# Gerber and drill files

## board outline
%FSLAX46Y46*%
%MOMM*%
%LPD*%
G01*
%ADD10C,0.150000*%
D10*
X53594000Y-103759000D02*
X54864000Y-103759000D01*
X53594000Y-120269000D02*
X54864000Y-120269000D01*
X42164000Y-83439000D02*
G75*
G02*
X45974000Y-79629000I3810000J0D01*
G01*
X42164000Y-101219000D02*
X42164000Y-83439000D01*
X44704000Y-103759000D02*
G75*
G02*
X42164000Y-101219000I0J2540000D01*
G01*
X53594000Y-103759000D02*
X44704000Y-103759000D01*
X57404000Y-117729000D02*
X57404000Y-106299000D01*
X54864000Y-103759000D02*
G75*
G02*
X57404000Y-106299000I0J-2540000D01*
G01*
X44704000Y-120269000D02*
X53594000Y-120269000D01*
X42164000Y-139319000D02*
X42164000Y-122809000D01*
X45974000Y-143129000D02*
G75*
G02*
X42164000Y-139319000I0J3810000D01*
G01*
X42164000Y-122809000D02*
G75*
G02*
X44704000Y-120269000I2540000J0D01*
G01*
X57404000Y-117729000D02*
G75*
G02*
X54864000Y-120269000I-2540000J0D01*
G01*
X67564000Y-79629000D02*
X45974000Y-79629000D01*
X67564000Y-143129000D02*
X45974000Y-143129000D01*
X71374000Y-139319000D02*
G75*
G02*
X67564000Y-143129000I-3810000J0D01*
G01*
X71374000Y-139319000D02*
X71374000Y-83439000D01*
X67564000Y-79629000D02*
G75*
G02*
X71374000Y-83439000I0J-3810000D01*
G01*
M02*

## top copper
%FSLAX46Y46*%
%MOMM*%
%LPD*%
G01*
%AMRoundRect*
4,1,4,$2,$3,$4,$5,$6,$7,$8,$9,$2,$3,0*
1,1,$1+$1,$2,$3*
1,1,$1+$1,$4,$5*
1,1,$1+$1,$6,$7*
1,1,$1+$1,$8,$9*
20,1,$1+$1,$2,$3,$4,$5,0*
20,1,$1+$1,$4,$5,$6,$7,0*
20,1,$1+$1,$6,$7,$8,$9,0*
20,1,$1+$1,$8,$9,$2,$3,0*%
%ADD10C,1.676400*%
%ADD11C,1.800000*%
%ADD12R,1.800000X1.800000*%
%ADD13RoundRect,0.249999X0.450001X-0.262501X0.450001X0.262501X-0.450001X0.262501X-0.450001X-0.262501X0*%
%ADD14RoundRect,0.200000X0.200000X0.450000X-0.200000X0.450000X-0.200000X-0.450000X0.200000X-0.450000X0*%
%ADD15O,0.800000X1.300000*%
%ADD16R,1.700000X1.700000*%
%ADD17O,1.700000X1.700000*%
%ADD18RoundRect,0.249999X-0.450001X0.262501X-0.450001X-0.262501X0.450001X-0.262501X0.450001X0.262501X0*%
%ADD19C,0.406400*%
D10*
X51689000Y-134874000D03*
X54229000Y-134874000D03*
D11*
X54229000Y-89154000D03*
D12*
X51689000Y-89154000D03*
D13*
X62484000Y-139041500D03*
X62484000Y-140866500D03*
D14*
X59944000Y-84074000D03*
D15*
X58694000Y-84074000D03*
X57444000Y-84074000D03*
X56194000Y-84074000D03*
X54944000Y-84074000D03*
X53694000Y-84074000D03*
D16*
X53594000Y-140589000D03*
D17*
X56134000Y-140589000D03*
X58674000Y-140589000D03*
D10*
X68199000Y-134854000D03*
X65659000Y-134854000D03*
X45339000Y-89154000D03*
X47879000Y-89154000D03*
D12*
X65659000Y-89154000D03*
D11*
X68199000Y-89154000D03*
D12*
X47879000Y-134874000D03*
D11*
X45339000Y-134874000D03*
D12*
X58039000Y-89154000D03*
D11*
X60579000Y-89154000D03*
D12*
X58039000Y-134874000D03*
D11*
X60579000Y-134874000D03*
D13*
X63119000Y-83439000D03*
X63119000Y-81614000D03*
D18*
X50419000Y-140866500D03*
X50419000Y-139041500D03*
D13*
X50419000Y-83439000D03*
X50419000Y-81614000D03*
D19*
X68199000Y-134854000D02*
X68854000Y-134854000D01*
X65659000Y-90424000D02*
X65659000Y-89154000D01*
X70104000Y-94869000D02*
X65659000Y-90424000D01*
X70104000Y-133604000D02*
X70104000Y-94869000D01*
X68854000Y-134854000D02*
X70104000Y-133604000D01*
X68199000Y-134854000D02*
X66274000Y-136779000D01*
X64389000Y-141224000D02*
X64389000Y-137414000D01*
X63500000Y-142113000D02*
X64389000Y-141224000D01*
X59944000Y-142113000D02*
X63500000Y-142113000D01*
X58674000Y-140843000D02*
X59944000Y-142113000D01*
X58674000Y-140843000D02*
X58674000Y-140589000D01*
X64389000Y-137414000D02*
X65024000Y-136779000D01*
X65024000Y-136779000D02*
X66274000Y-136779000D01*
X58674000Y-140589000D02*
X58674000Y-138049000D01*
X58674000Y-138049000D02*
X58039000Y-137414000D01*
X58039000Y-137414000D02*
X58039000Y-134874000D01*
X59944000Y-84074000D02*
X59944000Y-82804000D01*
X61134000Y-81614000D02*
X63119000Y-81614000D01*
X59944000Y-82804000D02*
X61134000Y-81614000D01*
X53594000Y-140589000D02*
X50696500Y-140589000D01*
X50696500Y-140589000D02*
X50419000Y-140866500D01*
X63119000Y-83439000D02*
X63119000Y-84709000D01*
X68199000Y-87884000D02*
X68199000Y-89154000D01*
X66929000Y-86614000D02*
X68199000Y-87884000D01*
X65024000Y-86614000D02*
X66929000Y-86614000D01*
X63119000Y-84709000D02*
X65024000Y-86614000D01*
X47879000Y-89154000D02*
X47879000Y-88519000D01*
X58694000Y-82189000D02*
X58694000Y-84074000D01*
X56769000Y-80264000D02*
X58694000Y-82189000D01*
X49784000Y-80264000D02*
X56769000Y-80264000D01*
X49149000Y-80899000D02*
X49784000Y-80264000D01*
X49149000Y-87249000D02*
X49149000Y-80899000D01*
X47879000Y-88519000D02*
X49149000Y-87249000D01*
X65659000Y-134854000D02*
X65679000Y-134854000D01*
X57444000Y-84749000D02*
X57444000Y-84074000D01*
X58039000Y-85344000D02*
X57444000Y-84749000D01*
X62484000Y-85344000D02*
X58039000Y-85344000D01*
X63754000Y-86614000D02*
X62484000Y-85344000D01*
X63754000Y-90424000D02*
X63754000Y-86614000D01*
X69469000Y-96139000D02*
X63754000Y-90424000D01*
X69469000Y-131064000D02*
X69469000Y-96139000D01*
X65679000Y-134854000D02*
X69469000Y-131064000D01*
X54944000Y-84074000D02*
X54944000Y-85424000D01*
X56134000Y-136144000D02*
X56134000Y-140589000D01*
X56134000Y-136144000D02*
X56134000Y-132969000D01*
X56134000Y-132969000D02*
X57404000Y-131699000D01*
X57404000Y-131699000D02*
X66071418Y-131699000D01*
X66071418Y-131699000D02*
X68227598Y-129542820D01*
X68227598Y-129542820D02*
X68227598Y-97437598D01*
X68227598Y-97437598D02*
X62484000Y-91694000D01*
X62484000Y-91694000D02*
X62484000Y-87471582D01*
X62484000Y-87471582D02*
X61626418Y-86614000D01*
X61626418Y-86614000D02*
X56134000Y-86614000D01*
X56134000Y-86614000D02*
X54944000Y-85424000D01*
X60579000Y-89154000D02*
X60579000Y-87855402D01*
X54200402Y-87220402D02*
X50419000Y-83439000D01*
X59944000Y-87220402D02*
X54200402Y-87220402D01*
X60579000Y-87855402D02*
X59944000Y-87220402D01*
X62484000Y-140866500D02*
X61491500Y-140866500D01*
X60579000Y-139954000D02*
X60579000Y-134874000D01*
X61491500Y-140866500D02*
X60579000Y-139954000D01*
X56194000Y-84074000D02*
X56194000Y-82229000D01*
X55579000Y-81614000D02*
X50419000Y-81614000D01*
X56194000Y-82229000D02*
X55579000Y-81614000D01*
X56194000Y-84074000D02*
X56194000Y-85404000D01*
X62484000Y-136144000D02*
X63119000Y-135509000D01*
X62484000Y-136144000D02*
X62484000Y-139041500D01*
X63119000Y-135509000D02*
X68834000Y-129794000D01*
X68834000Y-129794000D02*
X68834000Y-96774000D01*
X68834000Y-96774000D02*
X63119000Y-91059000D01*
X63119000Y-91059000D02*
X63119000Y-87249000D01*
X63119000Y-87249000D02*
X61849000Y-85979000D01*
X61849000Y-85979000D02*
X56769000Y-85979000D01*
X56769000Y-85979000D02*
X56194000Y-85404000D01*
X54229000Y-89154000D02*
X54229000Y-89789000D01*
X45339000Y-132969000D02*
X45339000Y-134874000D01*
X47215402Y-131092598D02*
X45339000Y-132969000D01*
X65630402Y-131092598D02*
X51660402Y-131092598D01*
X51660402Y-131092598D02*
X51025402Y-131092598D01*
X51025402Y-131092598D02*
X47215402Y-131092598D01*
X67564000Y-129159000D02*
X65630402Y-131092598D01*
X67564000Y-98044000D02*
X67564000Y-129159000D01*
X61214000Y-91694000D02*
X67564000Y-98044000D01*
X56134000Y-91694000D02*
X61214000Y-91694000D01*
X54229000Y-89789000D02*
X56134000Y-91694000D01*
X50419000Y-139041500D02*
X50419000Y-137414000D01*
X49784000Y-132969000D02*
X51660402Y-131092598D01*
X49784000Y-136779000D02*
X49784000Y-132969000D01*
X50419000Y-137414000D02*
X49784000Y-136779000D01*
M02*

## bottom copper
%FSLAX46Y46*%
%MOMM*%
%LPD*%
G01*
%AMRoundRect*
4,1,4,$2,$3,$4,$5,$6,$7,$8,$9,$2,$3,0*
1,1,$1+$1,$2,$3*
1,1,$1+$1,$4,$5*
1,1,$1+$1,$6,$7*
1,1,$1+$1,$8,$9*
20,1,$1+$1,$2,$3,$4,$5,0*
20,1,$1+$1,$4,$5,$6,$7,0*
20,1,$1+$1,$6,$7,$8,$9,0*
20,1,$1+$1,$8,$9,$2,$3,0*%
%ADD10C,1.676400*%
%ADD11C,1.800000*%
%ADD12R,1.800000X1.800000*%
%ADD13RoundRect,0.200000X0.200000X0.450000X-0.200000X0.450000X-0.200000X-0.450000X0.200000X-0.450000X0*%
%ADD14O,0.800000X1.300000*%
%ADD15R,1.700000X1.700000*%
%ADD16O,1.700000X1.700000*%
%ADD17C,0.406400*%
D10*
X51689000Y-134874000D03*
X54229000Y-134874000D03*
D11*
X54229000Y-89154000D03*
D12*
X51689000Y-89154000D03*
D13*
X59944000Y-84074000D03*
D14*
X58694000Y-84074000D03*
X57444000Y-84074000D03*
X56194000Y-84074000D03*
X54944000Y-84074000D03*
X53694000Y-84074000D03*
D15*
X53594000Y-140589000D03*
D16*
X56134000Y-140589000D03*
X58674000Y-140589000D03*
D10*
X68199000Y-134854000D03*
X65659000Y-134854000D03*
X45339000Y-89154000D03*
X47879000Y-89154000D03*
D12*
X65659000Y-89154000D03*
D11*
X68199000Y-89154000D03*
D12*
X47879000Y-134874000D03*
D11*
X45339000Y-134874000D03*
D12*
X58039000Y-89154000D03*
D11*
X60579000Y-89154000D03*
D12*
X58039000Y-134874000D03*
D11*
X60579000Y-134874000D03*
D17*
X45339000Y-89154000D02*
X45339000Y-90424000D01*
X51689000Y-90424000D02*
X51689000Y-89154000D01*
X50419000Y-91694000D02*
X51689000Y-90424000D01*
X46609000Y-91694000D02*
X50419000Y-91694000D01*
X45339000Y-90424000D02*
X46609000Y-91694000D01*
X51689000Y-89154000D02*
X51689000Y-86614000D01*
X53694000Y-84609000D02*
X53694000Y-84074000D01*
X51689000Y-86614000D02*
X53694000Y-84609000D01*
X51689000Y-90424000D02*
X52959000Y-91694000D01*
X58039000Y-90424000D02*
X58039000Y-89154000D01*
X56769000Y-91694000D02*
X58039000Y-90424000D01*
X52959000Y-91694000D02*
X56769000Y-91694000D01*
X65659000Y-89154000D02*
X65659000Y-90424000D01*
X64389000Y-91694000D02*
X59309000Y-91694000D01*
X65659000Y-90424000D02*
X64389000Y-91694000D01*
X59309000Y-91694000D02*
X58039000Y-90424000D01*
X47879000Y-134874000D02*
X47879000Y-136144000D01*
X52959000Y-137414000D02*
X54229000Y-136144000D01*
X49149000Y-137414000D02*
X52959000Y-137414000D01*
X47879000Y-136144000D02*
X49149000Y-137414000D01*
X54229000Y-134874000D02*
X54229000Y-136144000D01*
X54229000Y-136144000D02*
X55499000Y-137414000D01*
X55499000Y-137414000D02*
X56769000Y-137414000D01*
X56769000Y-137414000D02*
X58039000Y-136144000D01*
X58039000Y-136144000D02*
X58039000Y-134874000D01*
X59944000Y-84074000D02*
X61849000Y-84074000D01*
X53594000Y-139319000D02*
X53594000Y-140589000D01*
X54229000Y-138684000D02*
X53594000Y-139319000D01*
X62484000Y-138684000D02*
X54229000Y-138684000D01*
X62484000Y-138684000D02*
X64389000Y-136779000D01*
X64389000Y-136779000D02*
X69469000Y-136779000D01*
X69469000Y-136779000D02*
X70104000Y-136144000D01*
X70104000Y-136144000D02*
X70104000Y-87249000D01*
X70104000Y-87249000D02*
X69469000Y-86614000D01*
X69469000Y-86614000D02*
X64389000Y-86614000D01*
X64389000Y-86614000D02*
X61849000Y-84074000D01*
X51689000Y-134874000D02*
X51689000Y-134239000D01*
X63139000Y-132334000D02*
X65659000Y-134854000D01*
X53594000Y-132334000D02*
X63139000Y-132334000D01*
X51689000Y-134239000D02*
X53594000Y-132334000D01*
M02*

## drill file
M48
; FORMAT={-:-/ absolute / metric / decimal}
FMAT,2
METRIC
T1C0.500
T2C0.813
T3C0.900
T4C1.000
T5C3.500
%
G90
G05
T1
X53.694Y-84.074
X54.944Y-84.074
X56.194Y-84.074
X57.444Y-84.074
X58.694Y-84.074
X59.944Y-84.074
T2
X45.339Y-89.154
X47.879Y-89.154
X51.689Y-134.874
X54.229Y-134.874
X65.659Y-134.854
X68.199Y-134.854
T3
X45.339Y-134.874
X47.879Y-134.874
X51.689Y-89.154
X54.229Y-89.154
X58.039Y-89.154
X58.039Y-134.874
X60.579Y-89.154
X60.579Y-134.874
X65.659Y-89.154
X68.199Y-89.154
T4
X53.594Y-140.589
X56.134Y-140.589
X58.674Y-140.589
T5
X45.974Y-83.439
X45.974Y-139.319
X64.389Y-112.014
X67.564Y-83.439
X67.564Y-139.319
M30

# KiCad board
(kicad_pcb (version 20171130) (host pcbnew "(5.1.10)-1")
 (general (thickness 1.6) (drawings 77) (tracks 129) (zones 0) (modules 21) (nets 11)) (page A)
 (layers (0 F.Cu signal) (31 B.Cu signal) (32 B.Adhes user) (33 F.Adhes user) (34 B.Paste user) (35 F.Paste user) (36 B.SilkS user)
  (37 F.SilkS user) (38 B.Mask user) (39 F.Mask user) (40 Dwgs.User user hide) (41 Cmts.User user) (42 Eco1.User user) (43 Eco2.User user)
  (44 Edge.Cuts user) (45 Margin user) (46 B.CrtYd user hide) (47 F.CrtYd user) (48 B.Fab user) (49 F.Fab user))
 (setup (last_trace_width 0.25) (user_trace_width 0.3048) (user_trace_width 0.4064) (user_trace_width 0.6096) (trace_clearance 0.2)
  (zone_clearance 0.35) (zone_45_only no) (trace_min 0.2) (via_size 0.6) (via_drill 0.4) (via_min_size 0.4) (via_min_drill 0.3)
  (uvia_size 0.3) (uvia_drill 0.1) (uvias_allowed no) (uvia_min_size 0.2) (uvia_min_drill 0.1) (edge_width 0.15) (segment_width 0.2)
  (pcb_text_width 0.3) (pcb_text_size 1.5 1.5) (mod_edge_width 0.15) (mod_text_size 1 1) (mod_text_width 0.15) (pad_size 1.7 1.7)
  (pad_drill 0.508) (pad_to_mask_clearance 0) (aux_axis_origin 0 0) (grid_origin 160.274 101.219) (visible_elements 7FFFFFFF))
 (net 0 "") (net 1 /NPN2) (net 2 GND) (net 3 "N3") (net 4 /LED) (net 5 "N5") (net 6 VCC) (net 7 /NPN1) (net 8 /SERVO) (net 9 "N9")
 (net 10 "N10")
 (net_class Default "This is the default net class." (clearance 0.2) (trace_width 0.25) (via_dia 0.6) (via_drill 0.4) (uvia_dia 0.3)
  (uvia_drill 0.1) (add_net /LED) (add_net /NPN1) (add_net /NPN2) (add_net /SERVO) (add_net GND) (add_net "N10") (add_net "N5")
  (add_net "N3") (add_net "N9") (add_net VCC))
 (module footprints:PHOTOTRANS (layer F.Cu) (at 52.959 134.874 180)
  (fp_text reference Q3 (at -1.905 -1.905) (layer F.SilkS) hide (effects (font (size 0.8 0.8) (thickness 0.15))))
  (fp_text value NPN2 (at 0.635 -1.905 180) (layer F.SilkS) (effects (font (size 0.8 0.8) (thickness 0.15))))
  (pad 1 thru_hole circle (at 1.27 0 225) (size 1.6764 1.6764) (drill 0.8128) (layers *.Cu *.Mask F.SilkS) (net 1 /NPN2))
  (pad 2 thru_hole circle (at -1.27 0 180) (size 1.6764 1.6764) (drill 0.8128) (layers *.Cu *.Mask F.SilkS) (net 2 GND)))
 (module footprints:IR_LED (layer F.Cu) (at 51.689 89.154)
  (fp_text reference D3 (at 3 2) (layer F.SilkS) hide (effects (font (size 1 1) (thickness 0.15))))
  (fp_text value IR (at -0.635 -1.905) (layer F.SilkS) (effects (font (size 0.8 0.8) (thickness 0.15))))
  (pad 2 thru_hole circle (at 2.54 0) (size 1.8 1.8) (drill 0.9) (layers *.Cu *.Mask) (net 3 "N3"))
  (pad 1 thru_hole rect (at 0 0) (size 1.8 1.8) (drill 0.9) (layers *.Cu *.Mask) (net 2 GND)))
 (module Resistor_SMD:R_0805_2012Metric (layer F.Cu) (at 62.484 139.954 90)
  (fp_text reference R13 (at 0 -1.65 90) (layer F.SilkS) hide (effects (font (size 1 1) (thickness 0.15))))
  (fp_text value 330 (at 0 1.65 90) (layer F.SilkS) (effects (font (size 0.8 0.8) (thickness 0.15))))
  (pad 2 smd roundrect (at 0.9125 0 90) (size 1.025 1.4) (layers F.Cu F.Paste F.Mask) (roundrect_rratio 0.2439014634146341) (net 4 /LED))
  (pad 1 smd roundrect (at -0.9125 0 90) (size 1.025 1.4) (layers F.Cu F.Paste F.Mask) (roundrect_rratio 0.2439014634146341) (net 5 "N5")))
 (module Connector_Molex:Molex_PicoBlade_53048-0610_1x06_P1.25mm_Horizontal (layer F.Cu) (at 59.944 84.074 180)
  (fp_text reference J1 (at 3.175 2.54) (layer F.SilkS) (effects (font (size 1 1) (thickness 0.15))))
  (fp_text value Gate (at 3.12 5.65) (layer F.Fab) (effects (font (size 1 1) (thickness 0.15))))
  (pad 1 thru_hole roundrect (at 0 0 180) (size 0.8 1.3) (drill 0.5) (layers *.Cu *.Mask) (roundrect_rratio 0.25) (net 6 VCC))
  (pad 2 thru_hole oval (at 1.25 0 180) (size 0.8 1.3) (drill 0.5) (layers *.Cu *.Mask) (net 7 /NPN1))
  (pad 3 thru_hole oval (at 2.5 0 180) (size 0.8 1.3) (drill 0.5) (layers *.Cu *.Mask) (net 1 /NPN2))
  (pad 4 thru_hole oval (at 3.75 0 180) (size 0.8 1.3) (drill 0.5) (layers *.Cu *.Mask) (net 4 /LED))
  (pad 5 thru_hole oval (at 5 0 180) (size 0.8 1.3) (drill 0.5) (layers *.Cu *.Mask) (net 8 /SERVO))
  (pad 6 thru_hole oval (at 6.25 0 180) (size 0.8 1.3) (drill 0.5) (layers *.Cu *.Mask) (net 2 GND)))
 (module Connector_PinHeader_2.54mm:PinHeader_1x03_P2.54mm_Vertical (layer B.Cu) (at 53.594 140.589 270)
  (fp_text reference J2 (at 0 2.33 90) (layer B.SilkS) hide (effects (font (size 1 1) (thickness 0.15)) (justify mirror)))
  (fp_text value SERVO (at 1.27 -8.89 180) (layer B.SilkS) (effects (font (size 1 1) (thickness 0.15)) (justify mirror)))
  (pad 1 thru_hole rect (at 0 0 270) (size 1.7 1.7) (drill 1) (layers *.Cu *.Mask) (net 6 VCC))
  (pad 2 thru_hole oval (at 0 -2.54 270) (size 1.7 1.7) (drill 1) (layers *.Cu *.Mask) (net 8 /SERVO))
  (pad 3 thru_hole oval (at 0 -5.08 270) (size 1.7 1.7) (drill 1) (layers *.Cu *.Mask) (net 2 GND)))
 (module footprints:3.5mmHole (layer F.Cu) (at 67.564 139.319)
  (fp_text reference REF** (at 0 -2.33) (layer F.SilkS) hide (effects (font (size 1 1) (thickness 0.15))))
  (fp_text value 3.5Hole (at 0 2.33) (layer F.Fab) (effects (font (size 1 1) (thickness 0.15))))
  (pad "" np_thru_hole circle (at 0 0) (size 3.5 3.5) (drill 3.5) (layers *.Cu)))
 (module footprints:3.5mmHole (layer F.Cu) (at 67.564 83.439)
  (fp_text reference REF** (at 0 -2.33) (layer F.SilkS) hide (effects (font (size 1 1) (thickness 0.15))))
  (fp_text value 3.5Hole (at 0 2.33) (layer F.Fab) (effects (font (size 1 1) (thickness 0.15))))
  (pad "" np_thru_hole circle (at 0 0) (size 3.5 3.5) (drill 3.5) (layers *.Cu)))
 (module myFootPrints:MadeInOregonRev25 (layer F.Cu) (at 47.879 95.504)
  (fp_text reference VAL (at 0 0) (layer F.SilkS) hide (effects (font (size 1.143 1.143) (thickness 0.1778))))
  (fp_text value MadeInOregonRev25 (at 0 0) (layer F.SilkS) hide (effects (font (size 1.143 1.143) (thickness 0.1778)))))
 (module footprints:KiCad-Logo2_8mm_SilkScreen (layer B.Cu) (at 58.674 124.714 180)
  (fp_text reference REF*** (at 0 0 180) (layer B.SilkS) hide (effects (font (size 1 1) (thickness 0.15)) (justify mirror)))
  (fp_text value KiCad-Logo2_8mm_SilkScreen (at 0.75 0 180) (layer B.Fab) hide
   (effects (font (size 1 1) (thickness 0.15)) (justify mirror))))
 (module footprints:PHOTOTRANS (layer F.Cu) (at 66.929 134.854 180)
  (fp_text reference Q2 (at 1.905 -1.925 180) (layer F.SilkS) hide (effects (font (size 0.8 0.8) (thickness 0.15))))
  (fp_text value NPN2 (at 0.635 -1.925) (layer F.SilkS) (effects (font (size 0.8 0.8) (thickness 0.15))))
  (pad 2 thru_hole circle (at -1.27 0 180) (size 1.6764 1.6764) (drill 0.8128) (layers *.Cu *.Mask F.SilkS) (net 2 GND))
  (pad 1 thru_hole circle (at 1.27 0 225) (size 1.6764 1.6764) (drill 0.8128) (layers *.Cu *.Mask F.SilkS) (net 1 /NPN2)))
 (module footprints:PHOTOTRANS (layer F.Cu) (at 46.609 89.154)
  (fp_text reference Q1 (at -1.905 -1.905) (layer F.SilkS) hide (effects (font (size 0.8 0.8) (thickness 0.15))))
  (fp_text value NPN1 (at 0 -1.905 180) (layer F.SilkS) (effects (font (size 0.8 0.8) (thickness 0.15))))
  (pad 2 thru_hole circle (at -1.27 0) (size 1.6764 1.6764) (drill 0.8128) (layers *.Cu *.Mask F.SilkS) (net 2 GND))
  (pad 1 thru_hole circle (at 1.27 0 45) (size 1.6764 1.6764) (drill 0.8128) (layers *.Cu *.Mask F.SilkS) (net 7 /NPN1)))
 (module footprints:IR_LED (layer F.Cu) (at 65.659 89.154)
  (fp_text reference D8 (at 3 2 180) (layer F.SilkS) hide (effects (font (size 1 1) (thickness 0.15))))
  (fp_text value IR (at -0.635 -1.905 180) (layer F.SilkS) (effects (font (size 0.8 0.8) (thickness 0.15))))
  (pad 1 thru_hole rect (at 0 0) (size 1.8 1.8) (drill 0.9) (layers *.Cu *.Mask) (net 2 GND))
  (pad 2 thru_hole circle (at 2.54 0) (size 1.8 1.8) (drill 0.9) (layers *.Cu *.Mask) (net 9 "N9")))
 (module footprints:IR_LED (layer F.Cu) (at 47.879 134.874 180)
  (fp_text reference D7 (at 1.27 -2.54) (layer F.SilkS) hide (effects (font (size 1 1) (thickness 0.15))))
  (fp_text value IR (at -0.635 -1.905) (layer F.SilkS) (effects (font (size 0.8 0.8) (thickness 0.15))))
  (pad 1 thru_hole rect (at 0 0 180) (size 1.8 1.8) (drill 0.9) (layers *.Cu *.Mask) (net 2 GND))
  (pad 2 thru_hole circle (at 2.54 0 180) (size 1.8 1.8) (drill 0.9) (layers *.Cu *.Mask) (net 3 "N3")))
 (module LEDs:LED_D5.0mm (layer F.Cu) (at 58.039 89.154)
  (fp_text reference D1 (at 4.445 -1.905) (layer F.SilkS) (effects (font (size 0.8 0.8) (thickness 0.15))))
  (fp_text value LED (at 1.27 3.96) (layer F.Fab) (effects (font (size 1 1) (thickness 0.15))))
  (pad 1 thru_hole rect (at 0 0) (size 1.8 1.8) (drill 0.9) (layers *.Cu *.Mask) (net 2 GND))
  (pad 2 thru_hole circle (at 2.54 0) (size 1.8 1.8) (drill 0.9) (layers *.Cu *.Mask) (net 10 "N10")))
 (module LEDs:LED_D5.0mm (layer F.Cu) (at 58.039 134.874)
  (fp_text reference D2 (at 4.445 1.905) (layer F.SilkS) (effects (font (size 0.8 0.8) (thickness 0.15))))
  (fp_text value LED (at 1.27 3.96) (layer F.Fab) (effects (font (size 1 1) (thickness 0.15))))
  (pad 1 thru_hole rect (at 0 0) (size 1.8 1.8) (drill 0.9) (layers *.Cu *.Mask) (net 2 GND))
  (pad 2 thru_hole circle (at 2.54 0) (size 1.8 1.8) (drill 0.9) (layers *.Cu *.Mask) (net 5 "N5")))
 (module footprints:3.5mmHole (layer F.Cu) (at 64.389 112.014)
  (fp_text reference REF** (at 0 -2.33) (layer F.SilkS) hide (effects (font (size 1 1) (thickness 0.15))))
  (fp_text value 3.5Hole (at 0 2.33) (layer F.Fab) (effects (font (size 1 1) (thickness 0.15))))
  (pad "" np_thru_hole circle (at 0 0) (size 3.5 3.5) (drill 3.5) (layers *.Cu)))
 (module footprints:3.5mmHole (layer F.Cu) (at 45.974 139.319)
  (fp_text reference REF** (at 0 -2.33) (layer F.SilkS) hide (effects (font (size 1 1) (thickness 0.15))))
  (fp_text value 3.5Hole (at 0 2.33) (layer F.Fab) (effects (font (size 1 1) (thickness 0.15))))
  (pad "" np_thru_hole circle (at 0 0) (size 3.5 3.5) (drill 3.5) (layers *.Cu)))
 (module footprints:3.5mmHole (layer F.Cu) (at 45.974 83.439)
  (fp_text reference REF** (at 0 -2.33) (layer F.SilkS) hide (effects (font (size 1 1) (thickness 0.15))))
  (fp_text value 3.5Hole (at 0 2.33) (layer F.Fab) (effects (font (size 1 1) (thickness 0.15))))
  (pad "" np_thru_hole circle (at 0 0) (size 3.5 3.5) (drill 3.5) (layers *.Cu)))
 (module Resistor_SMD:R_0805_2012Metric (layer F.Cu) (at 63.119 82.5265 90)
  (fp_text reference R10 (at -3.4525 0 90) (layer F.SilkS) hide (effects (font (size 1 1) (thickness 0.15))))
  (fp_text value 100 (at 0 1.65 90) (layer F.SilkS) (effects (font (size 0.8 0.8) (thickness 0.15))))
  (pad 1 smd roundrect (at -0.9125 0 90) (size 1.025 1.4) (layers F.Cu F.Paste F.Mask) (roundrect_rratio 0.2439014634146341) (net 9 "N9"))
  (pad 2 smd roundrect (at 0.9125 0 90) (size 1.025 1.4) (layers F.Cu F.Paste F.Mask) (roundrect_rratio 0.2439014634146341) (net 6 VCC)))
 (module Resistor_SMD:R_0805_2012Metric (layer F.Cu) (at 50.419 139.954 270)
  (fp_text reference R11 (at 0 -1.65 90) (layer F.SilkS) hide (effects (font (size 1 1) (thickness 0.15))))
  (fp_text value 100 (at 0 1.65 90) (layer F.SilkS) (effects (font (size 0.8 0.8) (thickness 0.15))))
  (pad 2 smd roundrect (at 0.9125 0 270) (size 1.025 1.4) (layers F.Cu F.Paste F.Mask) (roundrect_rratio 0.2439014634146341) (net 6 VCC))
  (pad 1 smd roundrect (at -0.9125 0 270) (size 1.025 1.4) (layers F.Cu F.Paste F.Mask) (roundrect_rratio 0.2439014634146341) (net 3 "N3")))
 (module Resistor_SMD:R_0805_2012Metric (layer F.Cu) (at 50.419 82.5265 90)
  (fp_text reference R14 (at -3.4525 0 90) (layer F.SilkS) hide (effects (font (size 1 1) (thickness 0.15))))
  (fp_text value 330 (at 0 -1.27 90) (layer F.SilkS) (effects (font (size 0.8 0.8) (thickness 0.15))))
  (pad 1 smd roundrect (at -0.9125 0 90) (size 1.025 1.4) (layers F.Cu F.Paste F.Mask) (roundrect_rratio 0.2439014634146341) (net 10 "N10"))
  (pad 2 smd roundrect (at 0.9125 0 90) (size 1.025 1.4) (layers F.Cu F.Paste F.Mask) (roundrect_rratio 0.2439014634146341) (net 4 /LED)))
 (gr_line (start 53.594 103.759) (end 54.864 103.759) (angle 90) (layer Edge.Cuts) (width 0.15))
 (gr_line (start 53.594 120.269) (end 54.864 120.269) (angle 90) (layer Edge.Cuts) (width 0.15))
 (gr_arc (start 45.974 83.439) (end 42.164 83.439) (angle 90) (layer Edge.Cuts) (width 0.15))
 (gr_line (start 42.164 101.219) (end 42.164 83.439) (angle 90) (layer Edge.Cuts) (width 0.15))
 (gr_arc (start 44.704 101.219) (end 44.704 103.759) (angle 90) (layer Edge.Cuts) (width 0.15))
 (gr_line (start 53.594 103.759) (end 44.704 103.759) (angle 90) (layer Edge.Cuts) (width 0.15))
 (gr_line (start 57.404 117.729) (end 57.404 106.299) (angle 90) (layer Edge.Cuts) (width 0.15))
 (gr_arc (start 54.864 106.299) (end 54.864 103.759) (angle 90) (layer Edge.Cuts) (width 0.15))
 (gr_line (start 44.704 120.269) (end 53.594 120.269) (angle 90) (layer Edge.Cuts) (width 0.15))
 (gr_line (start 42.164 139.319) (end 42.164 122.809) (angle 90) (layer Edge.Cuts) (width 0.15))
 (gr_arc (start 45.974 139.319) (end 45.974 143.129) (angle 90) (layer Edge.Cuts) (width 0.15))
 (gr_arc (start 44.704 122.809) (end 42.164 122.809) (angle 90) (layer Edge.Cuts) (width 0.15))
 (gr_arc (start 54.864 117.729) (end 57.404 117.729) (angle 90) (layer Edge.Cuts) (width 0.15))
 (gr_line (start 67.564 79.629) (end 45.974 79.629) (angle 90) (layer Edge.Cuts) (width 0.15))
 (gr_line (start 67.564 143.129) (end 45.974 143.129) (angle 90) (layer Edge.Cuts) (width 0.15))
 (gr_arc (start 67.564 139.319) (end 71.374 139.319) (angle 90) (layer Edge.Cuts) (width 0.15))
 (gr_line (start 71.374 139.319) (end 71.374 83.439) (angle 90) (layer Edge.Cuts) (width 0.15))
 (gr_arc (start 67.564 83.439) (end 67.564 79.629) (angle 90) (layer Edge.Cuts) (width 0.15))
 (segment (start 45.339 89.154) (end 45.339 90.424) (width 0.4064) (layer B.Cu) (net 2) (status 400000))
 (segment (start 51.689 90.424) (end 51.689 89.154) (width 0.4064) (layer B.Cu) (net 2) (status 800000))
 (segment (start 50.419 91.694) (end 51.689 90.424) (width 0.4064) (layer B.Cu) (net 2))
 (segment (start 46.609 91.694) (end 50.419 91.694) (width 0.4064) (layer B.Cu) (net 2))
 (segment (start 45.339 90.424) (end 46.609 91.694) (width 0.4064) (layer B.Cu) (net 2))
 (segment (start 51.689 89.154) (end 51.689 86.614) (width 0.4064) (layer B.Cu) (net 2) (status 400000))
 (segment (start 53.694 84.609) (end 53.694 84.074) (width 0.4064) (layer B.Cu) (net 2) (status C00000))
 (segment (start 51.689 86.614) (end 53.694 84.609) (width 0.4064) (layer B.Cu) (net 2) (status 800000))
 (segment (start 51.689 90.424) (end 52.959 91.694) (width 0.4064) (layer B.Cu) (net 2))
 (segment (start 58.039 90.424) (end 58.039 89.154) (width 0.4064) (layer B.Cu) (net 2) (status 800000))
 (segment (start 56.769 91.694) (end 58.039 90.424) (width 0.4064) (layer B.Cu) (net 2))
 (segment (start 52.959 91.694) (end 56.769 91.694) (width 0.4064) (layer B.Cu) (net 2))
 (segment (start 65.659 89.154) (end 65.659 90.424) (width 0.4064) (layer B.Cu) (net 2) (status 400000))
 (segment (start 64.389 91.694) (end 59.309 91.694) (width 0.4064) (layer B.Cu) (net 2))
 (segment (start 65.659 90.424) (end 64.389 91.694) (width 0.4064) (layer B.Cu) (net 2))
 (segment (start 59.309 91.694) (end 58.039 90.424) (width 0.4064) (layer B.Cu) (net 2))
 (segment (start 47.879 134.874) (end 47.879 136.144) (width 0.4064) (layer B.Cu) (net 2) (status 400000))
 (segment (start 52.959 137.414) (end 54.229 136.144) (width 0.4064) (layer B.Cu) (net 2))
 (segment (start 49.149 137.414) (end 52.959 137.414) (width 0.4064) (layer B.Cu) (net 2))
 (segment (start 47.879 136.144) (end 49.149 137.414) (width 0.4064) (layer B.Cu) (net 2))
 (segment (start 54.229 134.874) (end 54.229 136.144) (width 0.4064) (layer B.Cu) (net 2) (status 400000))
 (segment (start 54.229 136.144) (end 55.499 137.414) (width 0.4064) (layer B.Cu) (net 2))
 (segment (start 55.499 137.414) (end 56.769 137.414) (width 0.4064) (layer B.Cu) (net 2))
 (segment (start 56.769 137.414) (end 58.039 136.144) (width 0.4064) (layer B.Cu) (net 2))
 (segment (start 58.039 136.144) (end 58.039 134.874) (width 0.4064) (layer B.Cu) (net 2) (status 800000))
 (segment (start 68.199 134.854) (end 68.854 134.854) (width 0.4064) (layer F.Cu) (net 2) (status C00000))
 (segment (start 65.659 90.424) (end 65.659 89.154) (width 0.4064) (layer F.Cu) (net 2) (status 800000))
 (segment (start 70.104 94.869) (end 65.659 90.424) (width 0.4064) (layer F.Cu) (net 2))
 (segment (start 70.104 133.604) (end 70.104 94.869) (width 0.4064) (layer F.Cu) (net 2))
 (segment (start 68.854 134.854) (end 70.104 133.604) (width 0.4064) (layer F.Cu) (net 2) (status 400000))
 (segment (start 68.199 134.854) (end 66.274 136.779) (width 0.4064) (layer F.Cu) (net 2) (status 400000))
 (segment (start 64.389 141.224) (end 64.389 137.414) (width 0.4064) (layer F.Cu) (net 2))
 (segment (start 63.5 142.113) (end 64.389 141.224) (width 0.4064) (layer F.Cu) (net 2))
 (segment (start 59.944 142.113) (end 63.5 142.113) (width 0.4064) (layer F.Cu) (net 2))
 (segment (start 58.674 140.843) (end 59.944 142.113) (width 0.4064) (layer F.Cu) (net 2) (status 400000))
 (segment (start 58.674 140.843) (end 58.674 140.589) (width 0.4064) (layer F.Cu) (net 2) (status C00000))
 (segment (start 64.389 137.414) (end 65.024 136.779) (width 0.4064) (layer F.Cu) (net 2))
 (segment (start 65.024 136.779) (end 66.274 136.779) (width 0.4064) (layer F.Cu) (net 2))
 (segment (start 58.674 140.589) (end 58.674 138.049) (width 0.4064) (layer F.Cu) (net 2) (status 400000))
 (segment (start 58.674 138.049) (end 58.039 137.414) (width 0.4064) (layer F.Cu) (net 2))
 (segment (start 58.039 137.414) (end 58.039 134.874) (width 0.4064) (layer F.Cu) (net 2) (status 800000))
 (segment (start 59.944 84.074) (end 61.849 84.074) (width 0.4064) (layer B.Cu) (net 6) (status 400000))
 (segment (start 53.594 139.319) (end 53.594 140.589) (width 0.4064) (layer B.Cu) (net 6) (status 800000))
 (segment (start 54.229 138.684) (end 53.594 139.319) (width 0.4064) (layer B.Cu) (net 6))
 (segment (start 62.484 138.684) (end 54.229 138.684) (width 0.4064) (layer B.Cu) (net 6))
 (segment (start 62.484 138.684) (end 64.389 136.779) (width 0.4064) (layer B.Cu) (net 6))
 (segment (start 64.389 136.779) (end 69.469 136.779) (width 0.4064) (layer B.Cu) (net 6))
 (segment (start 69.469 136.779) (end 70.104 136.144) (width 0.4064) (layer B.Cu) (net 6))
 (segment (start 70.104 136.144) (end 70.104 87.249) (width 0.4064) (layer B.Cu) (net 6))
 (segment (start 70.104 87.249) (end 69.469 86.614) (width 0.4064) (layer B.Cu) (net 6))
 (segment (start 69.469 86.614) (end 64.389 86.614) (width 0.4064) (layer B.Cu) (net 6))
 (segment (start 64.389 86.614) (end 61.849 84.074) (width 0.4064) (layer B.Cu) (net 6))
 (segment (start 59.944 84.074) (end 59.944 82.804) (width 0.4064) (layer F.Cu) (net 6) (status 400000))
 (segment (start 61.134 81.614) (end 63.119 81.614) (width 0.4064) (layer F.Cu) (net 6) (status 800000))
 (segment (start 59.944 82.804) (end 61.134 81.614) (width 0.4064) (layer F.Cu) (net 6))
 (segment (start 53.594 140.589) (end 50.6965 140.589) (width 0.4064) (layer F.Cu) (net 6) (status C00000))
 (segment (start 50.6965 140.589) (end 50.419 140.8665) (width 0.4064) (layer F.Cu) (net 6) (status C00000))
 (segment (start 63.119 83.439) (end 63.119 84.709) (width 0.4064) (layer F.Cu) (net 9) (status 400000))
 (segment (start 68.199 87.884) (end 68.199 89.154) (width 0.4064) (layer F.Cu) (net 9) (status 800000))
 (segment (start 66.929 86.614) (end 68.199 87.884) (width 0.4064) (layer F.Cu) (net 9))
 (segment (start 65.024 86.614) (end 66.929 86.614) (width 0.4064) (layer F.Cu) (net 9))
 (segment (start 63.119 84.709) (end 65.024 86.614) (width 0.4064) (layer F.Cu) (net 9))
 (segment (start 47.879 89.154) (end 47.879 88.519) (width 0.4064) (layer F.Cu) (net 7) (status C00000))
 (segment (start 58.694 82.189) (end 58.694 84.074) (width 0.4064) (layer F.Cu) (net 7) (status 800000))
 (segment (start 56.769 80.264) (end 58.694 82.189) (width 0.4064) (layer F.Cu) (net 7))
 (segment (start 49.784 80.264) (end 56.769 80.264) (width 0.4064) (layer F.Cu) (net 7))
 (segment (start 49.149 80.899) (end 49.784 80.264) (width 0.4064) (layer F.Cu) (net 7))
 (segment (start 49.149 87.249) (end 49.149 80.899) (width 0.4064) (layer F.Cu) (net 7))
 (segment (start 47.879 88.519) (end 49.149 87.249) (width 0.4064) (layer F.Cu) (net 7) (status 400000))
 (segment (start 65.659 134.854) (end 65.679 134.854) (width 0.4064) (layer F.Cu) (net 1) (status C00000))
 (segment (start 57.444 84.749) (end 57.444 84.074) (width 0.4064) (layer F.Cu) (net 1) (status 800000))
 (segment (start 58.039 85.344) (end 57.444 84.749) (width 0.4064) (layer F.Cu) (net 1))
 (segment (start 62.484 85.344) (end 58.039 85.344) (width 0.4064) (layer F.Cu) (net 1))
 (segment (start 63.754 86.614) (end 62.484 85.344) (width 0.4064) (layer F.Cu) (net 1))
 (segment (start 63.754 90.424) (end 63.754 86.614) (width 0.4064) (layer F.Cu) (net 1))
 (segment (start 69.469 96.139) (end 63.754 90.424) (width 0.4064) (layer F.Cu) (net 1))
 (segment (start 69.469 131.064) (end 69.469 96.139) (width 0.4064) (layer F.Cu) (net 1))
 (segment (start 65.679 134.854) (end 69.469 131.064) (width 0.4064) (layer F.Cu) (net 1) (status 400000))
 (segment (start 51.689 134.874) (end 51.689 134.239) (width 0.4064) (layer B.Cu) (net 1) (status C00000))
 (segment (start 63.139 132.334) (end 65.659 134.854) (width 0.4064) (layer B.Cu) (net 1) (status 800000))
 (segment (start 53.594 132.334) (end 63.139 132.334) (width 0.4064) (layer B.Cu) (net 1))
 (segment (start 51.689 134.239) (end 53.594 132.334) (width 0.4064) (layer B.Cu) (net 1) (status 400000))
 (segment (start 54.944 84.074) (end 54.944 85.424) (width 0.4064) (layer F.Cu) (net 8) (status 400000))
 (segment (start 56.134 136.144) (end 56.134 140.589) (width 0.4064) (layer F.Cu) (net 8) (status 800000))
 (segment (start 56.134 136.144) (end 56.134 132.969) (width 0.4064) (layer F.Cu) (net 8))
 (segment (start 56.134 132.969) (end 57.404 131.699) (width 0.4064) (layer F.Cu) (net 8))
 (segment (start 57.404 131.699) (end 66.071418 131.699) (width 0.4064) (layer F.Cu) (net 8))
 (segment (start 66.071418 131.699) (end 68.227598 129.54282) (width 0.4064) (layer F.Cu) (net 8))
 (segment (start 68.227598 129.54282) (end 68.227598 97.437598) (width 0.4064) (layer F.Cu) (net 8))
 (segment (start 68.227598 97.437598) (end 62.484 91.694) (width 0.4064) (layer F.Cu) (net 8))
 (segment (start 62.484 91.694) (end 62.484 87.471582) (width 0.4064) (layer F.Cu) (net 8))
 (segment (start 62.484 87.471582) (end 61.626418 86.614) (width 0.4064) (layer F.Cu) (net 8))
 (segment (start 61.626418 86.614) (end 56.134 86.614) (width 0.4064) (layer F.Cu) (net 8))
 (segment (start 56.134 86.614) (end 54.944 85.424) (width 0.4064) (layer F.Cu) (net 8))
 (segment (start 60.579 89.154) (end 60.579 87.855402) (width 0.4064) (layer F.Cu) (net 10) (status 400000))
 (segment (start 54.200402 87.220402) (end 50.419 83.439) (width 0.4064) (layer F.Cu) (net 10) (status 800000))
 (segment (start 59.944 87.220402) (end 54.200402 87.220402) (width 0.4064) (layer F.Cu) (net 10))
 (segment (start 60.579 87.855402) (end 59.944 87.220402) (width 0.4064) (layer F.Cu) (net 10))
 (segment (start 62.484 140.8665) (end 61.4915 140.8665) (width 0.4064) (layer F.Cu) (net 5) (status 400000))
 (segment (start 60.579 139.954) (end 60.579 134.874) (width 0.4064) (layer F.Cu) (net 5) (status 800000))
 (segment (start 61.4915 140.8665) (end 60.579 139.954) (width 0.4064) (layer F.Cu) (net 5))
 (segment (start 56.194 84.074) (end 56.194 82.229) (width 0.4064) (layer F.Cu) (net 4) (status 400000))
 (segment (start 55.579 81.614) (end 50.419 81.614) (width 0.4064) (layer F.Cu) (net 4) (status 800000))
 (segment (start 56.194 82.229) (end 55.579 81.614) (width 0.4064) (layer F.Cu) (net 4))
 (segment (start 56.194 84.074) (end 56.194 85.404) (width 0.4064) (layer F.Cu) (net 4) (status 400000))
 (segment (start 62.484 136.144) (end 63.119 135.509) (width 0.4064) (layer F.Cu) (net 4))
 (segment (start 62.484 136.144) (end 62.484 139.0415) (width 0.4064) (layer F.Cu) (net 4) (status 800000))
 (segment (start 63.119 135.509) (end 68.834 129.794) (width 0.4064) (layer F.Cu) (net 4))
 (segment (start 68.834 129.794) (end 68.834 96.774) (width 0.4064) (layer F.Cu) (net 4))
 (segment (start 68.834 96.774) (end 63.119 91.059) (width 0.4064) (layer F.Cu) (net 4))
 (segment (start 63.119 91.059) (end 63.119 87.249) (width 0.4064) (layer F.Cu) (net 4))
 (segment (start 63.119 87.249) (end 61.849 85.979) (width 0.4064) (layer F.Cu) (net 4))
 (segment (start 61.849 85.979) (end 56.769 85.979) (width 0.4064) (layer F.Cu) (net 4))
 (segment (start 56.769 85.979) (end 56.194 85.404) (width 0.4064) (layer F.Cu) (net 4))
 (segment (start 54.229 89.154) (end 54.229 89.789) (width 0.4064) (layer F.Cu) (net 3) (status C00000))
 (segment (start 45.339 132.969) (end 45.339 134.874) (width 0.4064) (layer F.Cu) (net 3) (status 800000))
 (segment (start 47.215402 131.092598) (end 45.339 132.969) (width 0.4064) (layer F.Cu) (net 3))
 (segment (start 65.630402 131.092598) (end 51.660402 131.092598) (width 0.4064) (layer F.Cu) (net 3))
 (segment (start 51.660402 131.092598) (end 51.025402 131.092598) (width 0.4064) (layer F.Cu) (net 3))
 (segment (start 51.025402 131.092598) (end 47.215402 131.092598) (width 0.4064) (layer F.Cu) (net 3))
 (segment (start 67.564 129.159) (end 65.630402 131.092598) (width 0.4064) (layer F.Cu) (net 3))
 (segment (start 67.564 98.044) (end 67.564 129.159) (width 0.4064) (layer F.Cu) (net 3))
 (segment (start 61.214 91.694) (end 67.564 98.044) (width 0.4064) (layer F.Cu) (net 3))
 (segment (start 56.134 91.694) (end 61.214 91.694) (width 0.4064) (layer F.Cu) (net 3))
 (segment (start 54.229 89.789) (end 56.134 91.694) (width 0.4064) (layer F.Cu) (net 3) (status 400000))
 (segment (start 50.419 139.0415) (end 50.419 137.414) (width 0.4064) (layer F.Cu) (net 3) (status 400000))
 (segment (start 49.784 132.969) (end 51.660402 131.092598) (width 0.4064) (layer F.Cu) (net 3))
 (segment (start 49.784 136.779) (end 49.784 132.969) (width 0.4064) (layer F.Cu) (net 3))
 (segment (start 50.419 137.414) (end 49.784 136.779) (width 0.4064) (layer F.Cu) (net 3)))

